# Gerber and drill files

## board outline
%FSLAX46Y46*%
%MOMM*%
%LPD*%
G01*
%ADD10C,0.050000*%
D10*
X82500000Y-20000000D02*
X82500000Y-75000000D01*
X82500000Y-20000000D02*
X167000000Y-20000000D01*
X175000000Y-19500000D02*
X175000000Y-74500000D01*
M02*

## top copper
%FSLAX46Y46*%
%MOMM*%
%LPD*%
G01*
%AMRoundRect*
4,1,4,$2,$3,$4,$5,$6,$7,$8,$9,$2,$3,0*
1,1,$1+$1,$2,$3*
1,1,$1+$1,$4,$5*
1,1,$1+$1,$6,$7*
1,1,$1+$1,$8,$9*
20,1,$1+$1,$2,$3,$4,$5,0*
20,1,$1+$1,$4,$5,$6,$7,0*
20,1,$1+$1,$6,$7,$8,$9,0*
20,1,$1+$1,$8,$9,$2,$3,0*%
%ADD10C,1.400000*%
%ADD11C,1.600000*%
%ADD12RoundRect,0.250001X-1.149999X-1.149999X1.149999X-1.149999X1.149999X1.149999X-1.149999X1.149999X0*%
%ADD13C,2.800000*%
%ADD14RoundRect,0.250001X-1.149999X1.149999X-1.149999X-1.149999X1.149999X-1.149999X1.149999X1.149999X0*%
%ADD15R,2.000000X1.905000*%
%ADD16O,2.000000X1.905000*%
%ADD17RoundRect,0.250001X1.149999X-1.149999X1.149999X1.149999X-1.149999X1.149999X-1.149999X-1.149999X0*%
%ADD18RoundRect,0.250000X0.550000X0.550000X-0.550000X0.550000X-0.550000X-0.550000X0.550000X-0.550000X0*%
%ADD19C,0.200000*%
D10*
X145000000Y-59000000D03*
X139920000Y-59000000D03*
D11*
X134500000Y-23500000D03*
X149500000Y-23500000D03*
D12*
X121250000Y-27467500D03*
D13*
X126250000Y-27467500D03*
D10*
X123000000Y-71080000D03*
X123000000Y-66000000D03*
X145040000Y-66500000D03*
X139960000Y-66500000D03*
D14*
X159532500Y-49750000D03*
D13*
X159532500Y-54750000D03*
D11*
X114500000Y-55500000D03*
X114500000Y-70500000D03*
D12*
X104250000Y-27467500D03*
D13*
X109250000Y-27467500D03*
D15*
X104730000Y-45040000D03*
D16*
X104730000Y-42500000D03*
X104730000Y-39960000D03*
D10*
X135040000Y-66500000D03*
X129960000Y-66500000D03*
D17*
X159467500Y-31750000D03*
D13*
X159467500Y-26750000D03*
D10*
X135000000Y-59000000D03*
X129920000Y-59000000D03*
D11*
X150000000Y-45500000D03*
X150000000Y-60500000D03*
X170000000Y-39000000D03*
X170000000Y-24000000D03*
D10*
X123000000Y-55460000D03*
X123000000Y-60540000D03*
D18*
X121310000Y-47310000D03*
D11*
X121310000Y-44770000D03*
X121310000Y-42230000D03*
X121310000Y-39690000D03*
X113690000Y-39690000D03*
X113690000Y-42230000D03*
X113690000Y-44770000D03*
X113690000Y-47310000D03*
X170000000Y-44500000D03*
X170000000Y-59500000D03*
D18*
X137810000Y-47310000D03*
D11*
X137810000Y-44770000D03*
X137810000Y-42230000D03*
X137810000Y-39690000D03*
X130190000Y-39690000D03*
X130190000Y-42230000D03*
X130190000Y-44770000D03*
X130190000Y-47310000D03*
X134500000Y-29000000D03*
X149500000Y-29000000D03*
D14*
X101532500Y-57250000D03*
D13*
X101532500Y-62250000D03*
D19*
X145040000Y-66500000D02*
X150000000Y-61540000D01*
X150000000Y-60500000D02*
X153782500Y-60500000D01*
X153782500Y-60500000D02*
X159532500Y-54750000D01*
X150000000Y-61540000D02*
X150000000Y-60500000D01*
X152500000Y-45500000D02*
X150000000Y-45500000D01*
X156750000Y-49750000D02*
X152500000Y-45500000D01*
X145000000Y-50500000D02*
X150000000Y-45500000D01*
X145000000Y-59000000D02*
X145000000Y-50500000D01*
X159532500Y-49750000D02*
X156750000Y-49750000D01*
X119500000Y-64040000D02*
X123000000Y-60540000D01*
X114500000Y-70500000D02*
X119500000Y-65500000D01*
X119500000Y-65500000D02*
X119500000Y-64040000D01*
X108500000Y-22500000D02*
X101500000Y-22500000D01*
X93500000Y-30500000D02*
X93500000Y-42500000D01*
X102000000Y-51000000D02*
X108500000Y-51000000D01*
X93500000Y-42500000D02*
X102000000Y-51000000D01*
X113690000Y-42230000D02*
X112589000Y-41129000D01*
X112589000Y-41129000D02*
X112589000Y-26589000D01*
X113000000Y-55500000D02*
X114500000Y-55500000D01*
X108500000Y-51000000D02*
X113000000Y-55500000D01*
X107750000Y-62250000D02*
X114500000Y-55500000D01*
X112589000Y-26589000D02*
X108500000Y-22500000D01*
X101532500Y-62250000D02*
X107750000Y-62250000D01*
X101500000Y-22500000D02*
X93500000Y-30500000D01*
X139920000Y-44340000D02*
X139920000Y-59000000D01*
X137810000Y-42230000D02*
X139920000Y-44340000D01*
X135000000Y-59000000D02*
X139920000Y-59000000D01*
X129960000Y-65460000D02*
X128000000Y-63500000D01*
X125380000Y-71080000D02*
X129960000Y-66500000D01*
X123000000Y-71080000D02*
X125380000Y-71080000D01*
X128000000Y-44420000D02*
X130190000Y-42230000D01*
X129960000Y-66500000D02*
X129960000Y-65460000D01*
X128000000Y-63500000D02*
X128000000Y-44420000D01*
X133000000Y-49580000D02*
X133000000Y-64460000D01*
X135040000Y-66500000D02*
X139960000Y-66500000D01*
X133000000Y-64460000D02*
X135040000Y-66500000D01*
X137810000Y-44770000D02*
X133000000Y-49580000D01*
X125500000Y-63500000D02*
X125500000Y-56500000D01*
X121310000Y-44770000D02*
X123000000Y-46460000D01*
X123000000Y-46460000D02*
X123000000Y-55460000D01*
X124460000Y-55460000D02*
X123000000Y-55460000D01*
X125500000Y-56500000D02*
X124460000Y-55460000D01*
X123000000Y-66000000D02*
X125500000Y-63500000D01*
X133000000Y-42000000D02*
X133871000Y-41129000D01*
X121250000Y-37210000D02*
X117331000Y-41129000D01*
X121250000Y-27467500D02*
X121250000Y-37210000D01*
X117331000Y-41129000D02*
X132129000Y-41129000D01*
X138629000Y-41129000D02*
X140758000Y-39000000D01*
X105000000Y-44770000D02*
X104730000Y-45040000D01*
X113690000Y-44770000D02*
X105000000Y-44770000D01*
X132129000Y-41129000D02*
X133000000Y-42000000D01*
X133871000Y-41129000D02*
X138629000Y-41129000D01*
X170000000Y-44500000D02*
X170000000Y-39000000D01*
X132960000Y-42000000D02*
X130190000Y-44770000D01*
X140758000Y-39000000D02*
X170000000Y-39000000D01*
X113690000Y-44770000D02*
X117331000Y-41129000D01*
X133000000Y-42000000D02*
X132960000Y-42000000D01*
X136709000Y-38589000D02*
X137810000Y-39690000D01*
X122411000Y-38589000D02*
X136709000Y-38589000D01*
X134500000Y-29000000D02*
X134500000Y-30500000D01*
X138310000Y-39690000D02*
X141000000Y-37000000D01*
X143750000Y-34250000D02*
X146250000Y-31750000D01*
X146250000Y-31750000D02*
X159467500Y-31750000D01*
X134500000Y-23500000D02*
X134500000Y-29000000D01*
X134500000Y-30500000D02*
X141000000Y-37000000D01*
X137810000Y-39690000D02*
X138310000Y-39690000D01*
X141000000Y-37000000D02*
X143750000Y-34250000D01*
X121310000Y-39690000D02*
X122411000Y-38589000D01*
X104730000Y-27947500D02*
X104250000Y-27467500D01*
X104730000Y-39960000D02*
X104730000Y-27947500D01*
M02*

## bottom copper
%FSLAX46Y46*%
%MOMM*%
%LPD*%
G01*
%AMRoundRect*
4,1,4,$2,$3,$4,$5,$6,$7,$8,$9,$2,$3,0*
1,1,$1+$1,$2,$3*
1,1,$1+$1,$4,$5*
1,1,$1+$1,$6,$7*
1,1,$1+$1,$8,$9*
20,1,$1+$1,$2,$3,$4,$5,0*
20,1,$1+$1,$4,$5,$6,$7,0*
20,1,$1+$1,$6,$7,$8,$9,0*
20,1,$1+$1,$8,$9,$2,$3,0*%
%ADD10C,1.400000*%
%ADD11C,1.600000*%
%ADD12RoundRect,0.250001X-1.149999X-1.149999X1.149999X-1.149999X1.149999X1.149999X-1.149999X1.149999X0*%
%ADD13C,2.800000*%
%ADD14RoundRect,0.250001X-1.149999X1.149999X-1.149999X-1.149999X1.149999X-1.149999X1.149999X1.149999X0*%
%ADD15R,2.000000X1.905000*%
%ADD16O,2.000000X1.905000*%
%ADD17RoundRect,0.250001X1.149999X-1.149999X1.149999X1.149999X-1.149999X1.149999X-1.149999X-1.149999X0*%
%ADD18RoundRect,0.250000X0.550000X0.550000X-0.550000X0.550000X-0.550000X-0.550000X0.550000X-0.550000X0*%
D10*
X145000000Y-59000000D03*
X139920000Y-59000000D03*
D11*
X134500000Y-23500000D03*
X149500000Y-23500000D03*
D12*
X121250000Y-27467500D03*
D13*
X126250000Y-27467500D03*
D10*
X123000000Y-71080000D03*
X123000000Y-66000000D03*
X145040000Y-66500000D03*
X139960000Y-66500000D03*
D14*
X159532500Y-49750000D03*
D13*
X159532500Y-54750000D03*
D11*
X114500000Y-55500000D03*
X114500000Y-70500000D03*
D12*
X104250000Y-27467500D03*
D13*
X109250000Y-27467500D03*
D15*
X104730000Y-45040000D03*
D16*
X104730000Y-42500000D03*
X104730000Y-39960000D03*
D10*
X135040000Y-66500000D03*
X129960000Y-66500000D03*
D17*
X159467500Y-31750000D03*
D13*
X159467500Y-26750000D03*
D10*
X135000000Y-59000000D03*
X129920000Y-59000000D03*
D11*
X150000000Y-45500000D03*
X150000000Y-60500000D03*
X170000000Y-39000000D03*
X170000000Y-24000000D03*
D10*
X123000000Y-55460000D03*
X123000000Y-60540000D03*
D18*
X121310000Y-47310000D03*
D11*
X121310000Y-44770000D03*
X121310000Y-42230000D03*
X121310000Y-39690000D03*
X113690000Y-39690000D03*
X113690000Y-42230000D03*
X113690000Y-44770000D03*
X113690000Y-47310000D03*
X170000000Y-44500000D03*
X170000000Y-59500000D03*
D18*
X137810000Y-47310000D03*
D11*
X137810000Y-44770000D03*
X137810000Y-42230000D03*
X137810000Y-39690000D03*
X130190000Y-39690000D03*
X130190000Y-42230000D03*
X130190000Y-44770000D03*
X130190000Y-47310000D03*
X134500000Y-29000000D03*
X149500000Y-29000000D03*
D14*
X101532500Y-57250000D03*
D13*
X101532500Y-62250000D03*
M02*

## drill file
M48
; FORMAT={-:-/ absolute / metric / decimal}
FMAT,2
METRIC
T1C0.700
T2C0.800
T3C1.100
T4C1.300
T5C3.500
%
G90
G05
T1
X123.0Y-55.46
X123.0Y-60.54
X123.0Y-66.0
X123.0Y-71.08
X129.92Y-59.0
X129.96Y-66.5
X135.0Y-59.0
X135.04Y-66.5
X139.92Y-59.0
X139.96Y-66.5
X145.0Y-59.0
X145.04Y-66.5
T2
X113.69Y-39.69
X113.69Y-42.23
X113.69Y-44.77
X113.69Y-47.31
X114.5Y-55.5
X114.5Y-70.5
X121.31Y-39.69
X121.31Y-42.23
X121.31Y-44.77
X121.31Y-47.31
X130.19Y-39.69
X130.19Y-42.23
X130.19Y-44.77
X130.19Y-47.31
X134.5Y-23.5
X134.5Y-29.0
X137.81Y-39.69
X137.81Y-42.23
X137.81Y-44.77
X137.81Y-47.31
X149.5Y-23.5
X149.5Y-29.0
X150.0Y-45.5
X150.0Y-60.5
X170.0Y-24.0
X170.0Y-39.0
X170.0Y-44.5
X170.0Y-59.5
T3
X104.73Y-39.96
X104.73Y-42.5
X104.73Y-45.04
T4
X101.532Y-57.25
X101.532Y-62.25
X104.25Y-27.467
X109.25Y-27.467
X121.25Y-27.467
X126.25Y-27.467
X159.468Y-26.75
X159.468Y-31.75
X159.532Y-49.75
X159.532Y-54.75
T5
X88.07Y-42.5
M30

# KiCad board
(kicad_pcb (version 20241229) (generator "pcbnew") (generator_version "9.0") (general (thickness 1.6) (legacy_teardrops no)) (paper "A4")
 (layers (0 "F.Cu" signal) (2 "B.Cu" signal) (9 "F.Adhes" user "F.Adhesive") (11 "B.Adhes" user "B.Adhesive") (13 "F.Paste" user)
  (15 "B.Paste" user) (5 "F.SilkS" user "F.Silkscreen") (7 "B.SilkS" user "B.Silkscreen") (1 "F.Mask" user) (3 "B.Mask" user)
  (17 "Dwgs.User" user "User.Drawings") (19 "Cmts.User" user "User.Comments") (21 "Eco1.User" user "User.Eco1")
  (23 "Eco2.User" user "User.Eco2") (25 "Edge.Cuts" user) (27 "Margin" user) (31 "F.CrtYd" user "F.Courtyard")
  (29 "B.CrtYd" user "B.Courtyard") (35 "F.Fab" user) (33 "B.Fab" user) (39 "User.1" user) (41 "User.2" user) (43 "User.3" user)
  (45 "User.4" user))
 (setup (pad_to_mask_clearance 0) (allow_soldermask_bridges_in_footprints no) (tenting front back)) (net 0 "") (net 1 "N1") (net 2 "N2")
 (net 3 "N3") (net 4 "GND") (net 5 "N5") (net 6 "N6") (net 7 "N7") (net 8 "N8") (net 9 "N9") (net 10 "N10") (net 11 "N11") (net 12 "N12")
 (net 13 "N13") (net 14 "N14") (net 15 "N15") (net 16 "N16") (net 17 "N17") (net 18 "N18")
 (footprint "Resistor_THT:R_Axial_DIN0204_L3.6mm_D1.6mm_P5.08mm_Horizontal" (layer "F.Cu") (at 145 59 180)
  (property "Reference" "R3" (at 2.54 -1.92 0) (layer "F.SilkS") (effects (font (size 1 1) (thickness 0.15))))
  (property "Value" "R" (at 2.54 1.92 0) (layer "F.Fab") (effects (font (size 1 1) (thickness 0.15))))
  (pad "1" thru_hole circle (at 0 0 180) (size 1.4 1.4) (drill 0.7) (layers "*.Cu" "*.Mask") (remove_unused_layers no) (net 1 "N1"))
  (pad "2" thru_hole circle (at 5.08 0 180) (size 1.4 1.4) (drill 0.7) (layers "*.Cu" "*.Mask") (remove_unused_layers no) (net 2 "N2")))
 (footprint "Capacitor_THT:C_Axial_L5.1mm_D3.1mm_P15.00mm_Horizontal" (layer "F.Cu") (at 134.5 23.5)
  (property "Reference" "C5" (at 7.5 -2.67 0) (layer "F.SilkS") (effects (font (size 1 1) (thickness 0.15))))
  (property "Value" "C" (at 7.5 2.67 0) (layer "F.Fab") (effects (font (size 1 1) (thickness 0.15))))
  (pad "1" thru_hole circle (at 0 0) (size 1.6 1.6) (drill 0.8) (layers "*.Cu" "*.Mask") (remove_unused_layers no) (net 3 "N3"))
  (pad "2" thru_hole circle (at 15 0) (size 1.6 1.6) (drill 0.8) (layers "*.Cu" "*.Mask") (remove_unused_layers no) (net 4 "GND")))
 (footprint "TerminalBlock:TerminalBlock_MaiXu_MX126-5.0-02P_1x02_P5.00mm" (layer "F.Cu") (at 121.25 27.4675)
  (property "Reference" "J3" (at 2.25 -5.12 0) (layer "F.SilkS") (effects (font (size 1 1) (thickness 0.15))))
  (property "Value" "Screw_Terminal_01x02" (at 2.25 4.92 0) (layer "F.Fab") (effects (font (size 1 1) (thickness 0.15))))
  (pad "1" thru_hole roundrect (at 0 0) (size 2.8 2.8) (drill 1.3) (layers "*.Cu" "*.Mask") (remove_unused_layers no)
   (roundrect_rratio 0.089286) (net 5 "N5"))
  (pad "2" thru_hole circle (at 5 0) (size 2.8 2.8) (drill 1.3) (layers "*.Cu" "*.Mask") (remove_unused_layers no) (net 4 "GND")))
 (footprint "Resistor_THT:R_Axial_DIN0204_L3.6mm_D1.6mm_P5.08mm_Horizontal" (layer "F.Cu") (at 123 71.08 90)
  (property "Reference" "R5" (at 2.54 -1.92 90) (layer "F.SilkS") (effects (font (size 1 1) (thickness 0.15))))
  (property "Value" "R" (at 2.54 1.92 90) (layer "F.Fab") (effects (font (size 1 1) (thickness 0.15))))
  (pad "1" thru_hole circle (at 0 0 90) (size 1.4 1.4) (drill 0.7) (layers "*.Cu" "*.Mask") (remove_unused_layers no) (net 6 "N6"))
  (pad "2" thru_hole circle (at 5.08 0 90) (size 1.4 1.4) (drill 0.7) (layers "*.Cu" "*.Mask") (remove_unused_layers no) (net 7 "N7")))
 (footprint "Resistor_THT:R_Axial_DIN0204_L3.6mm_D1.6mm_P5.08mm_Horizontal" (layer "F.Cu") (at 145.04 66.5 180)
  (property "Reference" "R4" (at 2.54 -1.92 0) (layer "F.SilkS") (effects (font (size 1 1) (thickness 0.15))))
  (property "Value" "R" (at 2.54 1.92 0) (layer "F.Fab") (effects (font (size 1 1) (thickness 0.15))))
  (pad "1" thru_hole circle (at 0 0 180) (size 1.4 1.4) (drill 0.7) (layers "*.Cu" "*.Mask") (remove_unused_layers no) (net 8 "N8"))
  (pad "2" thru_hole circle (at 5.08 0 180) (size 1.4 1.4) (drill 0.7) (layers "*.Cu" "*.Mask") (remove_unused_layers no) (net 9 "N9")))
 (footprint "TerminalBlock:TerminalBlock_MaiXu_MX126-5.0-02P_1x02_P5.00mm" (layer "F.Cu") (at 159.5325 49.75 -90)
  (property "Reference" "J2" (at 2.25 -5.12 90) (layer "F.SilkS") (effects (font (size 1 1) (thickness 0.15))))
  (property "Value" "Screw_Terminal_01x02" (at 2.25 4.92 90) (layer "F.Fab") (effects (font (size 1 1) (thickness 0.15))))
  (pad "1" thru_hole roundrect (at 0 0 270) (size 2.8 2.8) (drill 1.3) (layers "*.Cu" "*.Mask") (remove_unused_layers no)
   (roundrect_rratio 0.089286) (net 1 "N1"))
  (pad "2" thru_hole circle (at 5 0 270) (size 2.8 2.8) (drill 1.3) (layers "*.Cu" "*.Mask") (remove_unused_layers no) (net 8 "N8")))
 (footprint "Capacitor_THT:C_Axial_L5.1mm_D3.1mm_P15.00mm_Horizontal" (layer "F.Cu") (at 114.5 55.5 -90)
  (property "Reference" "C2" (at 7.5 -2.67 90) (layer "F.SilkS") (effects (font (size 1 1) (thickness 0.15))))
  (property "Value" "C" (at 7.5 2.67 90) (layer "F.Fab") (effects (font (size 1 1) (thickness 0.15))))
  (pad "1" thru_hole circle (at 0 0 270) (size 1.6 1.6) (drill 0.8) (layers "*.Cu" "*.Mask") (remove_unused_layers no) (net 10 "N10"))
  (pad "2" thru_hole circle (at 15 0 270) (size 1.6 1.6) (drill 0.8) (layers "*.Cu" "*.Mask") (remove_unused_layers no) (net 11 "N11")))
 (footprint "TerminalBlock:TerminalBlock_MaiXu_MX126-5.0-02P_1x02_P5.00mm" (layer "F.Cu") (at 104.25 27.4675)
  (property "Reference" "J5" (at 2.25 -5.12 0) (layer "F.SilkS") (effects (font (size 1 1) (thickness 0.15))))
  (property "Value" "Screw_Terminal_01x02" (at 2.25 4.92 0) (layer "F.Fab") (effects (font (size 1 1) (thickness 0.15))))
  (pad "1" thru_hole roundrect (at 0 0) (size 2.8 2.8) (drill 1.3) (layers "*.Cu" "*.Mask") (remove_unused_layers no)
   (roundrect_rratio 0.089286) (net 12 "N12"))
  (pad "2" thru_hole circle (at 5 0) (size 2.8 2.8) (drill 1.3) (layers "*.Cu" "*.Mask") (remove_unused_layers no) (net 4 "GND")))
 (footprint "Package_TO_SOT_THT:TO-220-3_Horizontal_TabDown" (layer "F.Cu") (at 104.73 45.04 90)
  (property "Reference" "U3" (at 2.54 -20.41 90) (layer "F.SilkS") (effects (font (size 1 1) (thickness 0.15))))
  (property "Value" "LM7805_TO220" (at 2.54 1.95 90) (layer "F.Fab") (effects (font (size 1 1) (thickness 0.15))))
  (pad "" np_thru_hole circle (at 2.54 -16.66 90) (size 3.5 3.5) (drill 3.5) (layers "*.Cu" "*.Mask"))
  (pad "1" thru_hole rect (at 0 0 90) (size 1.905 2) (drill 1.1) (layers "*.Cu" "*.Mask") (remove_unused_layers no) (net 5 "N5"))
  (pad "2" thru_hole oval (at 2.54 0 90) (size 1.905 2) (drill 1.1) (layers "*.Cu" "*.Mask") (remove_unused_layers no) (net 4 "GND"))
  (pad "3" thru_hole oval (at 5.08 0 90) (size 1.905 2) (drill 1.1) (layers "*.Cu" "*.Mask") (remove_unused_layers no) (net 12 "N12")))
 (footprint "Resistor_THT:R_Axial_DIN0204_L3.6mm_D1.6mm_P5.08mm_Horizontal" (layer "F.Cu") (at 135.04 66.5 180)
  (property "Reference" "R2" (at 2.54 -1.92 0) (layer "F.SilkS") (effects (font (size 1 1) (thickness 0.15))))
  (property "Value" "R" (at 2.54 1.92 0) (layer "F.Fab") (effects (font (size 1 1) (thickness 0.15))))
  (pad "1" thru_hole circle (at 0 0 180) (size 1.4 1.4) (drill 0.7) (layers "*.Cu" "*.Mask") (remove_unused_layers no) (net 9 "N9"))
  (pad "2" thru_hole circle (at 5.08 0 180) (size 1.4 1.4) (drill 0.7) (layers "*.Cu" "*.Mask") (remove_unused_layers no) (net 6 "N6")))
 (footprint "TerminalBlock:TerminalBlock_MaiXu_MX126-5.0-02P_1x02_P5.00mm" (layer "F.Cu") (at 159.4675 31.75 90)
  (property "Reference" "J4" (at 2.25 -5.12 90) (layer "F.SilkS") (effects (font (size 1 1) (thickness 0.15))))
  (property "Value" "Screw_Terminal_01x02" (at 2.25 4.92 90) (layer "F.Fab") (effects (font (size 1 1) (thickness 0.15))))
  (pad "1" thru_hole roundrect (at 0 0 90) (size 2.8 2.8) (drill 1.3) (layers "*.Cu" "*.Mask") (remove_unused_layers no)
   (roundrect_rratio 0.089286) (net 3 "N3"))
  (pad "2" thru_hole circle (at 5 0 90) (size 2.8 2.8) (drill 1.3) (layers "*.Cu" "*.Mask") (remove_unused_layers no) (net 4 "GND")))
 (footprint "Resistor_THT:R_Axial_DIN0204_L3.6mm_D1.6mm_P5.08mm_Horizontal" (layer "F.Cu") (at 135 59 180)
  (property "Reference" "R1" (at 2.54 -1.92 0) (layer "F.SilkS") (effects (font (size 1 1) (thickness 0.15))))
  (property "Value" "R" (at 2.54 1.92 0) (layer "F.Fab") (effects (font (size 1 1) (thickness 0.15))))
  (pad "1" thru_hole circle (at 0 0 180) (size 1.4 1.4) (drill 0.7) (layers "*.Cu" "*.Mask") (remove_unused_layers no) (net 2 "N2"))
  (pad "2" thru_hole circle (at 5.08 0 180) (size 1.4 1.4) (drill 0.7) (layers "*.Cu" "*.Mask") (remove_unused_layers no) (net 4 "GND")))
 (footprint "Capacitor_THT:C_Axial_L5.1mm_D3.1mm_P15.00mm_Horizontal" (layer "F.Cu") (at 150 45.5 -90)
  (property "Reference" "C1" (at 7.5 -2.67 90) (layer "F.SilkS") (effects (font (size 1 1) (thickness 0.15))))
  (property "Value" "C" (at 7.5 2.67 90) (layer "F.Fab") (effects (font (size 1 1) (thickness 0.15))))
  (pad "1" thru_hole circle (at 0 0 270) (size 1.6 1.6) (drill 0.8) (layers "*.Cu" "*.Mask") (remove_unused_layers no) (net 1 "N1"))
  (pad "2" thru_hole circle (at 15 0 270) (size 1.6 1.6) (drill 0.8) (layers "*.Cu" "*.Mask") (remove_unused_layers no) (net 8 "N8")))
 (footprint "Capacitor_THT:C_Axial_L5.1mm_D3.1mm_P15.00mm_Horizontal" (layer "F.Cu") (at 170 39 90)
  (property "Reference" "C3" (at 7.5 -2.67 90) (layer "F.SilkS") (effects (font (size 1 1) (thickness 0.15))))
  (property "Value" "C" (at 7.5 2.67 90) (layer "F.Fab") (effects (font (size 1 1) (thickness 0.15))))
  (pad "1" thru_hole circle (at 0 0 90) (size 1.6 1.6) (drill 0.8) (layers "*.Cu" "*.Mask") (remove_unused_layers no) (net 5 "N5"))
  (pad "2" thru_hole circle (at 15 0 90) (size 1.6 1.6) (drill 0.8) (layers "*.Cu" "*.Mask") (remove_unused_layers no) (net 4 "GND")))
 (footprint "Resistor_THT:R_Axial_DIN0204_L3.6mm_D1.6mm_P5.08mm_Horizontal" (layer "F.Cu") (at 123 55.46 -90)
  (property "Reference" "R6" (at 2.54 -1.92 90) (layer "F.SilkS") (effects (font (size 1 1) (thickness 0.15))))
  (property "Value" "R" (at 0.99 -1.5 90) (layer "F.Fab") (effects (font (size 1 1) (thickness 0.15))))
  (pad "1" thru_hole circle (at 0 0 270) (size 1.4 1.4) (drill 0.7) (layers "*.Cu" "*.Mask") (remove_unused_layers no) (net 7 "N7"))
  (pad "2" thru_hole circle (at 5.08 0 270) (size 1.4 1.4) (drill 0.7) (layers "*.Cu" "*.Mask") (remove_unused_layers no) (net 11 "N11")))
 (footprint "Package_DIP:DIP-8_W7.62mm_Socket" (layer "F.Cu") (at 121.31 47.31 180)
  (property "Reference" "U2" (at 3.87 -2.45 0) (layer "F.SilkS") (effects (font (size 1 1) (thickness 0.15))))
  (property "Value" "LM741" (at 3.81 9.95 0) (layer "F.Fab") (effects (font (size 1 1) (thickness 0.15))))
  (pad "1" thru_hole roundrect (at 0 0 180) (size 1.6 1.6) (drill 0.8) (layers "*.Cu" "*.Mask") (remove_unused_layers no)
   (roundrect_rratio 0.15625) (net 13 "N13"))
  (pad "2" thru_hole circle (at 0 2.54 180) (size 1.6 1.6) (drill 0.8) (layers "*.Cu" "*.Mask") (remove_unused_layers no) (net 7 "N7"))
  (pad "3" thru_hole circle (at 0 5.08 180) (size 1.6 1.6) (drill 0.8) (layers "*.Cu" "*.Mask") (remove_unused_layers no) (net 4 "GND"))
  (pad "4" thru_hole circle (at 0 7.62 180) (size 1.6 1.6) (drill 0.8) (layers "*.Cu" "*.Mask") (remove_unused_layers no) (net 3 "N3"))
  (pad "5" thru_hole circle (at 7.62 7.62 180) (size 1.6 1.6) (drill 0.8) (layers "*.Cu" "*.Mask") (remove_unused_layers no) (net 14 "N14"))
  (pad "6" thru_hole circle (at 7.62 5.08 180) (size 1.6 1.6) (drill 0.8) (layers "*.Cu" "*.Mask") (remove_unused_layers no) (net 10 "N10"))
  (pad "7" thru_hole circle (at 7.62 2.54 180) (size 1.6 1.6) (drill 0.8) (layers "*.Cu" "*.Mask") (remove_unused_layers no) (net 5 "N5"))
  (pad "8" thru_hole circle (at 7.62 0 180) (size 1.6 1.6) (drill 0.8) (layers "*.Cu" "*.Mask") (remove_unused_layers no) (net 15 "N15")))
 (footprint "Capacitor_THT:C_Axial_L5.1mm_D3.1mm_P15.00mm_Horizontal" (layer "F.Cu") (at 170 44.5 -90)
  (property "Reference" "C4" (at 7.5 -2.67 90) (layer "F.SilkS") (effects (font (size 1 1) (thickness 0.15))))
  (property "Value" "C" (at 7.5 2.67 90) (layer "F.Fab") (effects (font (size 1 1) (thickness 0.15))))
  (pad "1" thru_hole circle (at 0 0 270) (size 1.6 1.6) (drill 0.8) (layers "*.Cu" "*.Mask") (remove_unused_layers no) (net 5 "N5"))
  (pad "2" thru_hole circle (at 15 0 270) (size 1.6 1.6) (drill 0.8) (layers "*.Cu" "*.Mask") (remove_unused_layers no) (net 4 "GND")))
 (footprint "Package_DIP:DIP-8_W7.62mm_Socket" (layer "F.Cu") (at 137.81 47.31 180)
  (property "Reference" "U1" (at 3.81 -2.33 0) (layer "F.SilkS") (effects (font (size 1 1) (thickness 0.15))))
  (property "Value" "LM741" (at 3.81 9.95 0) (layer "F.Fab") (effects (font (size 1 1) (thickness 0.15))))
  (pad "1" thru_hole roundrect (at 0 0 180) (size 1.6 1.6) (drill 0.8) (layers "*.Cu" "*.Mask") (remove_unused_layers no)
   (roundrect_rratio 0.15625) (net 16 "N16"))
  (pad "2" thru_hole circle (at 0 2.54 180) (size 1.6 1.6) (drill 0.8) (layers "*.Cu" "*.Mask") (remove_unused_layers no) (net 9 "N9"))
  (pad "3" thru_hole circle (at 0 5.08 180) (size 1.6 1.6) (drill 0.8) (layers "*.Cu" "*.Mask") (remove_unused_layers no) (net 2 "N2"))
  (pad "4" thru_hole circle (at 0 7.62 180) (size 1.6 1.6) (drill 0.8) (layers "*.Cu" "*.Mask") (remove_unused_layers no) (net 3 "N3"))
  (pad "5" thru_hole circle (at 7.62 7.62 180) (size 1.6 1.6) (drill 0.8) (layers "*.Cu" "*.Mask") (remove_unused_layers no) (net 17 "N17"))
  (pad "6" thru_hole circle (at 7.62 5.08 180) (size 1.6 1.6) (drill 0.8) (layers "*.Cu" "*.Mask") (remove_unused_layers no) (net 6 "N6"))
  (pad "7" thru_hole circle (at 7.62 2.54 180) (size 1.6 1.6) (drill 0.8) (layers "*.Cu" "*.Mask") (remove_unused_layers no) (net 5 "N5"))
  (pad "8" thru_hole circle (at 7.62 0 180) (size 1.6 1.6) (drill 0.8) (layers "*.Cu" "*.Mask") (remove_unused_layers no) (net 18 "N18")))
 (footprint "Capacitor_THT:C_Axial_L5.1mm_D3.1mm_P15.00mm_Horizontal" (layer "F.Cu") (at 134.5 29)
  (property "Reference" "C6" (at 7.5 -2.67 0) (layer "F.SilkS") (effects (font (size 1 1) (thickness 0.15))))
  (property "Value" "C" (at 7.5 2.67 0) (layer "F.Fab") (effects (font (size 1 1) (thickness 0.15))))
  (pad "1" thru_hole circle (at 0 0) (size 1.6 1.6) (drill 0.8) (layers "*.Cu" "*.Mask") (remove_unused_layers no) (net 3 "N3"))
  (pad "2" thru_hole circle (at 15 0) (size 1.6 1.6) (drill 0.8) (layers "*.Cu" "*.Mask") (remove_unused_layers no) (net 4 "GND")))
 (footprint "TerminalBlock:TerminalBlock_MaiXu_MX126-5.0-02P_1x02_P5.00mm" (layer "F.Cu") (at 101.5325 57.25 -90)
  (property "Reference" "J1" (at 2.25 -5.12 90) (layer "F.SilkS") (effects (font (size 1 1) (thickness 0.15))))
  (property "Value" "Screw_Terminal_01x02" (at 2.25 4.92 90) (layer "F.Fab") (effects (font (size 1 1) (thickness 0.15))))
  (pad "1" thru_hole roundrect (at 0 0 270) (size 2.8 2.8) (drill 1.3) (layers "*.Cu" "*.Mask") (remove_unused_layers no)
   (roundrect_rratio 0.089286) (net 4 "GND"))
  (pad "2" thru_hole circle (at 5 0 270) (size 2.8 2.8) (drill 1.3) (layers "*.Cu" "*.Mask") (remove_unused_layers no) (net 10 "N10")))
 (gr_line (start 82.5 20) (end 82.5 75) (stroke (width 0.05) (type default)) (layer "Edge.Cuts"))
 (gr_line (start 82.5 20) (end 167 20) (stroke (width 0.05) (type default)) (layer "Edge.Cuts"))
 (gr_line (start 175 19.5) (end 175 74.5) (stroke (width 0.05) (type default)) (layer "Edge.Cuts"))
 (segment (start 145.04 66.5) (end 150 61.54) (width 0.2) (layer "F.Cu") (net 8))
 (segment (start 150 60.5) (end 153.7825 60.5) (width 0.2) (layer "F.Cu") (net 8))
 (segment (start 153.7825 60.5) (end 159.5325 54.75) (width 0.2) (layer "F.Cu") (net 8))
 (segment (start 150 61.54) (end 150 60.5) (width 0.2) (layer "F.Cu") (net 8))
 (segment (start 152.5 45.5) (end 150 45.5) (width 0.2) (layer "F.Cu") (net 1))
 (segment (start 156.75 49.75) (end 152.5 45.5) (width 0.2) (layer "F.Cu") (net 1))
 (segment (start 145 50.5) (end 150 45.5) (width 0.2) (layer "F.Cu") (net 1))
 (segment (start 145 59) (end 145 50.5) (width 0.2) (layer "F.Cu") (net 1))
 (segment (start 159.5325 49.75) (end 156.75 49.75) (width 0.2) (layer "F.Cu") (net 1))
 (segment (start 119.5 64.04) (end 123 60.54) (width 0.2) (layer "F.Cu") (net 11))
 (segment (start 114.5 70.5) (end 119.5 65.5) (width 0.2) (layer "F.Cu") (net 11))
 (segment (start 119.5 65.5) (end 119.5 64.04) (width 0.2) (layer "F.Cu") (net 11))
 (segment (start 108.5 22.5) (end 101.5 22.5) (width 0.2) (layer "F.Cu") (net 10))
 (segment (start 93.5 30.5) (end 93.5 42.5) (width 0.2) (layer "F.Cu") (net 10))
 (segment (start 102 51) (end 108.5 51) (width 0.2) (layer "F.Cu") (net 10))
 (segment (start 93.5 42.5) (end 102 51) (width 0.2) (layer "F.Cu") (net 10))
 (segment (start 113.69 42.23) (end 112.589 41.129) (width 0.2) (layer "F.Cu") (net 10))
 (segment (start 112.589 41.129) (end 112.589 26.589) (width 0.2) (layer "F.Cu") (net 10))
 (segment (start 113 55.5) (end 114.5 55.5) (width 0.2) (layer "F.Cu") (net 10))
 (segment (start 108.5 51) (end 113 55.5) (width 0.2) (layer "F.Cu") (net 10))
 (segment (start 107.75 62.25) (end 114.5 55.5) (width 0.2) (layer "F.Cu") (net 10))
 (segment (start 112.589 26.589) (end 108.5 22.5) (width 0.2) (layer "F.Cu") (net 10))
 (segment (start 101.5325 62.25) (end 107.75 62.25) (width 0.2) (layer "F.Cu") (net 10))
 (segment (start 101.5 22.5) (end 93.5 30.5) (width 0.2) (layer "F.Cu") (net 10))
 (segment (start 139.92 44.34) (end 139.92 59) (width 0.2) (layer "F.Cu") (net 2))
 (segment (start 137.81 42.23) (end 139.92 44.34) (width 0.2) (layer "F.Cu") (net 2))
 (segment (start 135 59) (end 139.92 59) (width 0.2) (layer "F.Cu") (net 2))
 (segment (start 129.96 65.46) (end 128 63.5) (width 0.2) (layer "F.Cu") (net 6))
 (segment (start 125.38 71.08) (end 129.96 66.5) (width 0.2) (layer "F.Cu") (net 6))
 (segment (start 123 71.08) (end 125.38 71.08) (width 0.2) (layer "F.Cu") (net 6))
 (segment (start 128 44.42) (end 130.19 42.23) (width 0.2) (layer "F.Cu") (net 6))
 (segment (start 129.96 66.5) (end 129.96 65.46) (width 0.2) (layer "F.Cu") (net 6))
 (segment (start 128 63.5) (end 128 44.42) (width 0.2) (layer "F.Cu") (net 6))
 (segment (start 133 49.58) (end 133 64.46) (width 0.2) (layer "F.Cu") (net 9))
 (segment (start 135.04 66.5) (end 139.96 66.5) (width 0.2) (layer "F.Cu") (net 9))
 (segment (start 133 64.46) (end 135.04 66.5) (width 0.2) (layer "F.Cu") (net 9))
 (segment (start 137.81 44.77) (end 133 49.58) (width 0.2) (layer "F.Cu") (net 9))
 (segment (start 125.5 63.5) (end 125.5 56.5) (width 0.2) (layer "F.Cu") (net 7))
 (segment (start 121.31 44.77) (end 123 46.46) (width 0.2) (layer "F.Cu") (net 7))
 (segment (start 123 46.46) (end 123 55.46) (width 0.2) (layer "F.Cu") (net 7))
 (segment (start 124.46 55.46) (end 123 55.46) (width 0.2) (layer "F.Cu") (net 7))
 (segment (start 125.5 56.5) (end 124.46 55.46) (width 0.2) (layer "F.Cu") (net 7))
 (segment (start 123 66) (end 125.5 63.5) (width 0.2) (layer "F.Cu") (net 7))
 (segment (start 133 42) (end 133.871 41.129) (width 0.2) (layer "F.Cu") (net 5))
 (segment (start 121.25 37.21) (end 117.331 41.129) (width 0.2) (layer "F.Cu") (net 5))
 (segment (start 121.25 27.4675) (end 121.25 37.21) (width 0.2) (layer "F.Cu") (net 5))
 (segment (start 117.331 41.129) (end 132.129 41.129) (width 0.2) (layer "F.Cu") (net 5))
 (segment (start 138.629 41.129) (end 140.758 39) (width 0.2) (layer "F.Cu") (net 5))
 (segment (start 105 44.77) (end 104.73 45.04) (width 0.2) (layer "F.Cu") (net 5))
 (segment (start 113.69 44.77) (end 105 44.77) (width 0.2) (layer "F.Cu") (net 5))
 (segment (start 132.129 41.129) (end 133 42) (width 0.2) (layer "F.Cu") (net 5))
 (segment (start 133.871 41.129) (end 138.629 41.129) (width 0.2) (layer "F.Cu") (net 5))
 (segment (start 170 44.5) (end 170 39) (width 0.2) (layer "F.Cu") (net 5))
 (segment (start 132.96 42) (end 130.19 44.77) (width 0.2) (layer "F.Cu") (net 5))
 (segment (start 140.758 39) (end 170 39) (width 0.2) (layer "F.Cu") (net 5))
 (segment (start 113.69 44.77) (end 117.331 41.129) (width 0.2) (layer "F.Cu") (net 5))
 (segment (start 133 42) (end 132.96 42) (width 0.2) (layer "F.Cu") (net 5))
 (segment (start 136.709 38.589) (end 137.81 39.69) (width 0.2) (layer "F.Cu") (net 3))
 (segment (start 122.411 38.589) (end 136.709 38.589) (width 0.2) (layer "F.Cu") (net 3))
 (segment (start 134.5 29) (end 134.5 30.5) (width 0.2) (layer "F.Cu") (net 3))
 (segment (start 138.31 39.69) (end 141 37) (width 0.2) (layer "F.Cu") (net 3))
 (segment (start 143.75 34.25) (end 146.25 31.75) (width 0.2) (layer "F.Cu") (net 3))
 (segment (start 146.25 31.75) (end 159.4675 31.75) (width 0.2) (layer "F.Cu") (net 3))
 (segment (start 134.5 23.5) (end 134.5 29) (width 0.2) (layer "F.Cu") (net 3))
 (segment (start 134.5 30.5) (end 141 37) (width 0.2) (layer "F.Cu") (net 3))
 (segment (start 137.81 39.69) (end 138.31 39.69) (width 0.2) (layer "F.Cu") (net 3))
 (segment (start 141 37) (end 143.75 34.25) (width 0.2) (layer "F.Cu") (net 3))
 (segment (start 121.31 39.69) (end 122.411 38.589) (width 0.2) (layer "F.Cu") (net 3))
 (segment (start 104.73 27.9475) (end 104.25 27.4675) (width 0.2) (layer "F.Cu") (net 12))
 (segment (start 104.73 39.96) (end 104.73 27.9475) (width 0.2) (layer "F.Cu") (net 12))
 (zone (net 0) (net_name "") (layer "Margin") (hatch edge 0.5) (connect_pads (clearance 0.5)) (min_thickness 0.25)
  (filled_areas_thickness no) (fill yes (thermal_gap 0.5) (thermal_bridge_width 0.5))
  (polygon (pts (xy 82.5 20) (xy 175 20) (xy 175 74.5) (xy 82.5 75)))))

